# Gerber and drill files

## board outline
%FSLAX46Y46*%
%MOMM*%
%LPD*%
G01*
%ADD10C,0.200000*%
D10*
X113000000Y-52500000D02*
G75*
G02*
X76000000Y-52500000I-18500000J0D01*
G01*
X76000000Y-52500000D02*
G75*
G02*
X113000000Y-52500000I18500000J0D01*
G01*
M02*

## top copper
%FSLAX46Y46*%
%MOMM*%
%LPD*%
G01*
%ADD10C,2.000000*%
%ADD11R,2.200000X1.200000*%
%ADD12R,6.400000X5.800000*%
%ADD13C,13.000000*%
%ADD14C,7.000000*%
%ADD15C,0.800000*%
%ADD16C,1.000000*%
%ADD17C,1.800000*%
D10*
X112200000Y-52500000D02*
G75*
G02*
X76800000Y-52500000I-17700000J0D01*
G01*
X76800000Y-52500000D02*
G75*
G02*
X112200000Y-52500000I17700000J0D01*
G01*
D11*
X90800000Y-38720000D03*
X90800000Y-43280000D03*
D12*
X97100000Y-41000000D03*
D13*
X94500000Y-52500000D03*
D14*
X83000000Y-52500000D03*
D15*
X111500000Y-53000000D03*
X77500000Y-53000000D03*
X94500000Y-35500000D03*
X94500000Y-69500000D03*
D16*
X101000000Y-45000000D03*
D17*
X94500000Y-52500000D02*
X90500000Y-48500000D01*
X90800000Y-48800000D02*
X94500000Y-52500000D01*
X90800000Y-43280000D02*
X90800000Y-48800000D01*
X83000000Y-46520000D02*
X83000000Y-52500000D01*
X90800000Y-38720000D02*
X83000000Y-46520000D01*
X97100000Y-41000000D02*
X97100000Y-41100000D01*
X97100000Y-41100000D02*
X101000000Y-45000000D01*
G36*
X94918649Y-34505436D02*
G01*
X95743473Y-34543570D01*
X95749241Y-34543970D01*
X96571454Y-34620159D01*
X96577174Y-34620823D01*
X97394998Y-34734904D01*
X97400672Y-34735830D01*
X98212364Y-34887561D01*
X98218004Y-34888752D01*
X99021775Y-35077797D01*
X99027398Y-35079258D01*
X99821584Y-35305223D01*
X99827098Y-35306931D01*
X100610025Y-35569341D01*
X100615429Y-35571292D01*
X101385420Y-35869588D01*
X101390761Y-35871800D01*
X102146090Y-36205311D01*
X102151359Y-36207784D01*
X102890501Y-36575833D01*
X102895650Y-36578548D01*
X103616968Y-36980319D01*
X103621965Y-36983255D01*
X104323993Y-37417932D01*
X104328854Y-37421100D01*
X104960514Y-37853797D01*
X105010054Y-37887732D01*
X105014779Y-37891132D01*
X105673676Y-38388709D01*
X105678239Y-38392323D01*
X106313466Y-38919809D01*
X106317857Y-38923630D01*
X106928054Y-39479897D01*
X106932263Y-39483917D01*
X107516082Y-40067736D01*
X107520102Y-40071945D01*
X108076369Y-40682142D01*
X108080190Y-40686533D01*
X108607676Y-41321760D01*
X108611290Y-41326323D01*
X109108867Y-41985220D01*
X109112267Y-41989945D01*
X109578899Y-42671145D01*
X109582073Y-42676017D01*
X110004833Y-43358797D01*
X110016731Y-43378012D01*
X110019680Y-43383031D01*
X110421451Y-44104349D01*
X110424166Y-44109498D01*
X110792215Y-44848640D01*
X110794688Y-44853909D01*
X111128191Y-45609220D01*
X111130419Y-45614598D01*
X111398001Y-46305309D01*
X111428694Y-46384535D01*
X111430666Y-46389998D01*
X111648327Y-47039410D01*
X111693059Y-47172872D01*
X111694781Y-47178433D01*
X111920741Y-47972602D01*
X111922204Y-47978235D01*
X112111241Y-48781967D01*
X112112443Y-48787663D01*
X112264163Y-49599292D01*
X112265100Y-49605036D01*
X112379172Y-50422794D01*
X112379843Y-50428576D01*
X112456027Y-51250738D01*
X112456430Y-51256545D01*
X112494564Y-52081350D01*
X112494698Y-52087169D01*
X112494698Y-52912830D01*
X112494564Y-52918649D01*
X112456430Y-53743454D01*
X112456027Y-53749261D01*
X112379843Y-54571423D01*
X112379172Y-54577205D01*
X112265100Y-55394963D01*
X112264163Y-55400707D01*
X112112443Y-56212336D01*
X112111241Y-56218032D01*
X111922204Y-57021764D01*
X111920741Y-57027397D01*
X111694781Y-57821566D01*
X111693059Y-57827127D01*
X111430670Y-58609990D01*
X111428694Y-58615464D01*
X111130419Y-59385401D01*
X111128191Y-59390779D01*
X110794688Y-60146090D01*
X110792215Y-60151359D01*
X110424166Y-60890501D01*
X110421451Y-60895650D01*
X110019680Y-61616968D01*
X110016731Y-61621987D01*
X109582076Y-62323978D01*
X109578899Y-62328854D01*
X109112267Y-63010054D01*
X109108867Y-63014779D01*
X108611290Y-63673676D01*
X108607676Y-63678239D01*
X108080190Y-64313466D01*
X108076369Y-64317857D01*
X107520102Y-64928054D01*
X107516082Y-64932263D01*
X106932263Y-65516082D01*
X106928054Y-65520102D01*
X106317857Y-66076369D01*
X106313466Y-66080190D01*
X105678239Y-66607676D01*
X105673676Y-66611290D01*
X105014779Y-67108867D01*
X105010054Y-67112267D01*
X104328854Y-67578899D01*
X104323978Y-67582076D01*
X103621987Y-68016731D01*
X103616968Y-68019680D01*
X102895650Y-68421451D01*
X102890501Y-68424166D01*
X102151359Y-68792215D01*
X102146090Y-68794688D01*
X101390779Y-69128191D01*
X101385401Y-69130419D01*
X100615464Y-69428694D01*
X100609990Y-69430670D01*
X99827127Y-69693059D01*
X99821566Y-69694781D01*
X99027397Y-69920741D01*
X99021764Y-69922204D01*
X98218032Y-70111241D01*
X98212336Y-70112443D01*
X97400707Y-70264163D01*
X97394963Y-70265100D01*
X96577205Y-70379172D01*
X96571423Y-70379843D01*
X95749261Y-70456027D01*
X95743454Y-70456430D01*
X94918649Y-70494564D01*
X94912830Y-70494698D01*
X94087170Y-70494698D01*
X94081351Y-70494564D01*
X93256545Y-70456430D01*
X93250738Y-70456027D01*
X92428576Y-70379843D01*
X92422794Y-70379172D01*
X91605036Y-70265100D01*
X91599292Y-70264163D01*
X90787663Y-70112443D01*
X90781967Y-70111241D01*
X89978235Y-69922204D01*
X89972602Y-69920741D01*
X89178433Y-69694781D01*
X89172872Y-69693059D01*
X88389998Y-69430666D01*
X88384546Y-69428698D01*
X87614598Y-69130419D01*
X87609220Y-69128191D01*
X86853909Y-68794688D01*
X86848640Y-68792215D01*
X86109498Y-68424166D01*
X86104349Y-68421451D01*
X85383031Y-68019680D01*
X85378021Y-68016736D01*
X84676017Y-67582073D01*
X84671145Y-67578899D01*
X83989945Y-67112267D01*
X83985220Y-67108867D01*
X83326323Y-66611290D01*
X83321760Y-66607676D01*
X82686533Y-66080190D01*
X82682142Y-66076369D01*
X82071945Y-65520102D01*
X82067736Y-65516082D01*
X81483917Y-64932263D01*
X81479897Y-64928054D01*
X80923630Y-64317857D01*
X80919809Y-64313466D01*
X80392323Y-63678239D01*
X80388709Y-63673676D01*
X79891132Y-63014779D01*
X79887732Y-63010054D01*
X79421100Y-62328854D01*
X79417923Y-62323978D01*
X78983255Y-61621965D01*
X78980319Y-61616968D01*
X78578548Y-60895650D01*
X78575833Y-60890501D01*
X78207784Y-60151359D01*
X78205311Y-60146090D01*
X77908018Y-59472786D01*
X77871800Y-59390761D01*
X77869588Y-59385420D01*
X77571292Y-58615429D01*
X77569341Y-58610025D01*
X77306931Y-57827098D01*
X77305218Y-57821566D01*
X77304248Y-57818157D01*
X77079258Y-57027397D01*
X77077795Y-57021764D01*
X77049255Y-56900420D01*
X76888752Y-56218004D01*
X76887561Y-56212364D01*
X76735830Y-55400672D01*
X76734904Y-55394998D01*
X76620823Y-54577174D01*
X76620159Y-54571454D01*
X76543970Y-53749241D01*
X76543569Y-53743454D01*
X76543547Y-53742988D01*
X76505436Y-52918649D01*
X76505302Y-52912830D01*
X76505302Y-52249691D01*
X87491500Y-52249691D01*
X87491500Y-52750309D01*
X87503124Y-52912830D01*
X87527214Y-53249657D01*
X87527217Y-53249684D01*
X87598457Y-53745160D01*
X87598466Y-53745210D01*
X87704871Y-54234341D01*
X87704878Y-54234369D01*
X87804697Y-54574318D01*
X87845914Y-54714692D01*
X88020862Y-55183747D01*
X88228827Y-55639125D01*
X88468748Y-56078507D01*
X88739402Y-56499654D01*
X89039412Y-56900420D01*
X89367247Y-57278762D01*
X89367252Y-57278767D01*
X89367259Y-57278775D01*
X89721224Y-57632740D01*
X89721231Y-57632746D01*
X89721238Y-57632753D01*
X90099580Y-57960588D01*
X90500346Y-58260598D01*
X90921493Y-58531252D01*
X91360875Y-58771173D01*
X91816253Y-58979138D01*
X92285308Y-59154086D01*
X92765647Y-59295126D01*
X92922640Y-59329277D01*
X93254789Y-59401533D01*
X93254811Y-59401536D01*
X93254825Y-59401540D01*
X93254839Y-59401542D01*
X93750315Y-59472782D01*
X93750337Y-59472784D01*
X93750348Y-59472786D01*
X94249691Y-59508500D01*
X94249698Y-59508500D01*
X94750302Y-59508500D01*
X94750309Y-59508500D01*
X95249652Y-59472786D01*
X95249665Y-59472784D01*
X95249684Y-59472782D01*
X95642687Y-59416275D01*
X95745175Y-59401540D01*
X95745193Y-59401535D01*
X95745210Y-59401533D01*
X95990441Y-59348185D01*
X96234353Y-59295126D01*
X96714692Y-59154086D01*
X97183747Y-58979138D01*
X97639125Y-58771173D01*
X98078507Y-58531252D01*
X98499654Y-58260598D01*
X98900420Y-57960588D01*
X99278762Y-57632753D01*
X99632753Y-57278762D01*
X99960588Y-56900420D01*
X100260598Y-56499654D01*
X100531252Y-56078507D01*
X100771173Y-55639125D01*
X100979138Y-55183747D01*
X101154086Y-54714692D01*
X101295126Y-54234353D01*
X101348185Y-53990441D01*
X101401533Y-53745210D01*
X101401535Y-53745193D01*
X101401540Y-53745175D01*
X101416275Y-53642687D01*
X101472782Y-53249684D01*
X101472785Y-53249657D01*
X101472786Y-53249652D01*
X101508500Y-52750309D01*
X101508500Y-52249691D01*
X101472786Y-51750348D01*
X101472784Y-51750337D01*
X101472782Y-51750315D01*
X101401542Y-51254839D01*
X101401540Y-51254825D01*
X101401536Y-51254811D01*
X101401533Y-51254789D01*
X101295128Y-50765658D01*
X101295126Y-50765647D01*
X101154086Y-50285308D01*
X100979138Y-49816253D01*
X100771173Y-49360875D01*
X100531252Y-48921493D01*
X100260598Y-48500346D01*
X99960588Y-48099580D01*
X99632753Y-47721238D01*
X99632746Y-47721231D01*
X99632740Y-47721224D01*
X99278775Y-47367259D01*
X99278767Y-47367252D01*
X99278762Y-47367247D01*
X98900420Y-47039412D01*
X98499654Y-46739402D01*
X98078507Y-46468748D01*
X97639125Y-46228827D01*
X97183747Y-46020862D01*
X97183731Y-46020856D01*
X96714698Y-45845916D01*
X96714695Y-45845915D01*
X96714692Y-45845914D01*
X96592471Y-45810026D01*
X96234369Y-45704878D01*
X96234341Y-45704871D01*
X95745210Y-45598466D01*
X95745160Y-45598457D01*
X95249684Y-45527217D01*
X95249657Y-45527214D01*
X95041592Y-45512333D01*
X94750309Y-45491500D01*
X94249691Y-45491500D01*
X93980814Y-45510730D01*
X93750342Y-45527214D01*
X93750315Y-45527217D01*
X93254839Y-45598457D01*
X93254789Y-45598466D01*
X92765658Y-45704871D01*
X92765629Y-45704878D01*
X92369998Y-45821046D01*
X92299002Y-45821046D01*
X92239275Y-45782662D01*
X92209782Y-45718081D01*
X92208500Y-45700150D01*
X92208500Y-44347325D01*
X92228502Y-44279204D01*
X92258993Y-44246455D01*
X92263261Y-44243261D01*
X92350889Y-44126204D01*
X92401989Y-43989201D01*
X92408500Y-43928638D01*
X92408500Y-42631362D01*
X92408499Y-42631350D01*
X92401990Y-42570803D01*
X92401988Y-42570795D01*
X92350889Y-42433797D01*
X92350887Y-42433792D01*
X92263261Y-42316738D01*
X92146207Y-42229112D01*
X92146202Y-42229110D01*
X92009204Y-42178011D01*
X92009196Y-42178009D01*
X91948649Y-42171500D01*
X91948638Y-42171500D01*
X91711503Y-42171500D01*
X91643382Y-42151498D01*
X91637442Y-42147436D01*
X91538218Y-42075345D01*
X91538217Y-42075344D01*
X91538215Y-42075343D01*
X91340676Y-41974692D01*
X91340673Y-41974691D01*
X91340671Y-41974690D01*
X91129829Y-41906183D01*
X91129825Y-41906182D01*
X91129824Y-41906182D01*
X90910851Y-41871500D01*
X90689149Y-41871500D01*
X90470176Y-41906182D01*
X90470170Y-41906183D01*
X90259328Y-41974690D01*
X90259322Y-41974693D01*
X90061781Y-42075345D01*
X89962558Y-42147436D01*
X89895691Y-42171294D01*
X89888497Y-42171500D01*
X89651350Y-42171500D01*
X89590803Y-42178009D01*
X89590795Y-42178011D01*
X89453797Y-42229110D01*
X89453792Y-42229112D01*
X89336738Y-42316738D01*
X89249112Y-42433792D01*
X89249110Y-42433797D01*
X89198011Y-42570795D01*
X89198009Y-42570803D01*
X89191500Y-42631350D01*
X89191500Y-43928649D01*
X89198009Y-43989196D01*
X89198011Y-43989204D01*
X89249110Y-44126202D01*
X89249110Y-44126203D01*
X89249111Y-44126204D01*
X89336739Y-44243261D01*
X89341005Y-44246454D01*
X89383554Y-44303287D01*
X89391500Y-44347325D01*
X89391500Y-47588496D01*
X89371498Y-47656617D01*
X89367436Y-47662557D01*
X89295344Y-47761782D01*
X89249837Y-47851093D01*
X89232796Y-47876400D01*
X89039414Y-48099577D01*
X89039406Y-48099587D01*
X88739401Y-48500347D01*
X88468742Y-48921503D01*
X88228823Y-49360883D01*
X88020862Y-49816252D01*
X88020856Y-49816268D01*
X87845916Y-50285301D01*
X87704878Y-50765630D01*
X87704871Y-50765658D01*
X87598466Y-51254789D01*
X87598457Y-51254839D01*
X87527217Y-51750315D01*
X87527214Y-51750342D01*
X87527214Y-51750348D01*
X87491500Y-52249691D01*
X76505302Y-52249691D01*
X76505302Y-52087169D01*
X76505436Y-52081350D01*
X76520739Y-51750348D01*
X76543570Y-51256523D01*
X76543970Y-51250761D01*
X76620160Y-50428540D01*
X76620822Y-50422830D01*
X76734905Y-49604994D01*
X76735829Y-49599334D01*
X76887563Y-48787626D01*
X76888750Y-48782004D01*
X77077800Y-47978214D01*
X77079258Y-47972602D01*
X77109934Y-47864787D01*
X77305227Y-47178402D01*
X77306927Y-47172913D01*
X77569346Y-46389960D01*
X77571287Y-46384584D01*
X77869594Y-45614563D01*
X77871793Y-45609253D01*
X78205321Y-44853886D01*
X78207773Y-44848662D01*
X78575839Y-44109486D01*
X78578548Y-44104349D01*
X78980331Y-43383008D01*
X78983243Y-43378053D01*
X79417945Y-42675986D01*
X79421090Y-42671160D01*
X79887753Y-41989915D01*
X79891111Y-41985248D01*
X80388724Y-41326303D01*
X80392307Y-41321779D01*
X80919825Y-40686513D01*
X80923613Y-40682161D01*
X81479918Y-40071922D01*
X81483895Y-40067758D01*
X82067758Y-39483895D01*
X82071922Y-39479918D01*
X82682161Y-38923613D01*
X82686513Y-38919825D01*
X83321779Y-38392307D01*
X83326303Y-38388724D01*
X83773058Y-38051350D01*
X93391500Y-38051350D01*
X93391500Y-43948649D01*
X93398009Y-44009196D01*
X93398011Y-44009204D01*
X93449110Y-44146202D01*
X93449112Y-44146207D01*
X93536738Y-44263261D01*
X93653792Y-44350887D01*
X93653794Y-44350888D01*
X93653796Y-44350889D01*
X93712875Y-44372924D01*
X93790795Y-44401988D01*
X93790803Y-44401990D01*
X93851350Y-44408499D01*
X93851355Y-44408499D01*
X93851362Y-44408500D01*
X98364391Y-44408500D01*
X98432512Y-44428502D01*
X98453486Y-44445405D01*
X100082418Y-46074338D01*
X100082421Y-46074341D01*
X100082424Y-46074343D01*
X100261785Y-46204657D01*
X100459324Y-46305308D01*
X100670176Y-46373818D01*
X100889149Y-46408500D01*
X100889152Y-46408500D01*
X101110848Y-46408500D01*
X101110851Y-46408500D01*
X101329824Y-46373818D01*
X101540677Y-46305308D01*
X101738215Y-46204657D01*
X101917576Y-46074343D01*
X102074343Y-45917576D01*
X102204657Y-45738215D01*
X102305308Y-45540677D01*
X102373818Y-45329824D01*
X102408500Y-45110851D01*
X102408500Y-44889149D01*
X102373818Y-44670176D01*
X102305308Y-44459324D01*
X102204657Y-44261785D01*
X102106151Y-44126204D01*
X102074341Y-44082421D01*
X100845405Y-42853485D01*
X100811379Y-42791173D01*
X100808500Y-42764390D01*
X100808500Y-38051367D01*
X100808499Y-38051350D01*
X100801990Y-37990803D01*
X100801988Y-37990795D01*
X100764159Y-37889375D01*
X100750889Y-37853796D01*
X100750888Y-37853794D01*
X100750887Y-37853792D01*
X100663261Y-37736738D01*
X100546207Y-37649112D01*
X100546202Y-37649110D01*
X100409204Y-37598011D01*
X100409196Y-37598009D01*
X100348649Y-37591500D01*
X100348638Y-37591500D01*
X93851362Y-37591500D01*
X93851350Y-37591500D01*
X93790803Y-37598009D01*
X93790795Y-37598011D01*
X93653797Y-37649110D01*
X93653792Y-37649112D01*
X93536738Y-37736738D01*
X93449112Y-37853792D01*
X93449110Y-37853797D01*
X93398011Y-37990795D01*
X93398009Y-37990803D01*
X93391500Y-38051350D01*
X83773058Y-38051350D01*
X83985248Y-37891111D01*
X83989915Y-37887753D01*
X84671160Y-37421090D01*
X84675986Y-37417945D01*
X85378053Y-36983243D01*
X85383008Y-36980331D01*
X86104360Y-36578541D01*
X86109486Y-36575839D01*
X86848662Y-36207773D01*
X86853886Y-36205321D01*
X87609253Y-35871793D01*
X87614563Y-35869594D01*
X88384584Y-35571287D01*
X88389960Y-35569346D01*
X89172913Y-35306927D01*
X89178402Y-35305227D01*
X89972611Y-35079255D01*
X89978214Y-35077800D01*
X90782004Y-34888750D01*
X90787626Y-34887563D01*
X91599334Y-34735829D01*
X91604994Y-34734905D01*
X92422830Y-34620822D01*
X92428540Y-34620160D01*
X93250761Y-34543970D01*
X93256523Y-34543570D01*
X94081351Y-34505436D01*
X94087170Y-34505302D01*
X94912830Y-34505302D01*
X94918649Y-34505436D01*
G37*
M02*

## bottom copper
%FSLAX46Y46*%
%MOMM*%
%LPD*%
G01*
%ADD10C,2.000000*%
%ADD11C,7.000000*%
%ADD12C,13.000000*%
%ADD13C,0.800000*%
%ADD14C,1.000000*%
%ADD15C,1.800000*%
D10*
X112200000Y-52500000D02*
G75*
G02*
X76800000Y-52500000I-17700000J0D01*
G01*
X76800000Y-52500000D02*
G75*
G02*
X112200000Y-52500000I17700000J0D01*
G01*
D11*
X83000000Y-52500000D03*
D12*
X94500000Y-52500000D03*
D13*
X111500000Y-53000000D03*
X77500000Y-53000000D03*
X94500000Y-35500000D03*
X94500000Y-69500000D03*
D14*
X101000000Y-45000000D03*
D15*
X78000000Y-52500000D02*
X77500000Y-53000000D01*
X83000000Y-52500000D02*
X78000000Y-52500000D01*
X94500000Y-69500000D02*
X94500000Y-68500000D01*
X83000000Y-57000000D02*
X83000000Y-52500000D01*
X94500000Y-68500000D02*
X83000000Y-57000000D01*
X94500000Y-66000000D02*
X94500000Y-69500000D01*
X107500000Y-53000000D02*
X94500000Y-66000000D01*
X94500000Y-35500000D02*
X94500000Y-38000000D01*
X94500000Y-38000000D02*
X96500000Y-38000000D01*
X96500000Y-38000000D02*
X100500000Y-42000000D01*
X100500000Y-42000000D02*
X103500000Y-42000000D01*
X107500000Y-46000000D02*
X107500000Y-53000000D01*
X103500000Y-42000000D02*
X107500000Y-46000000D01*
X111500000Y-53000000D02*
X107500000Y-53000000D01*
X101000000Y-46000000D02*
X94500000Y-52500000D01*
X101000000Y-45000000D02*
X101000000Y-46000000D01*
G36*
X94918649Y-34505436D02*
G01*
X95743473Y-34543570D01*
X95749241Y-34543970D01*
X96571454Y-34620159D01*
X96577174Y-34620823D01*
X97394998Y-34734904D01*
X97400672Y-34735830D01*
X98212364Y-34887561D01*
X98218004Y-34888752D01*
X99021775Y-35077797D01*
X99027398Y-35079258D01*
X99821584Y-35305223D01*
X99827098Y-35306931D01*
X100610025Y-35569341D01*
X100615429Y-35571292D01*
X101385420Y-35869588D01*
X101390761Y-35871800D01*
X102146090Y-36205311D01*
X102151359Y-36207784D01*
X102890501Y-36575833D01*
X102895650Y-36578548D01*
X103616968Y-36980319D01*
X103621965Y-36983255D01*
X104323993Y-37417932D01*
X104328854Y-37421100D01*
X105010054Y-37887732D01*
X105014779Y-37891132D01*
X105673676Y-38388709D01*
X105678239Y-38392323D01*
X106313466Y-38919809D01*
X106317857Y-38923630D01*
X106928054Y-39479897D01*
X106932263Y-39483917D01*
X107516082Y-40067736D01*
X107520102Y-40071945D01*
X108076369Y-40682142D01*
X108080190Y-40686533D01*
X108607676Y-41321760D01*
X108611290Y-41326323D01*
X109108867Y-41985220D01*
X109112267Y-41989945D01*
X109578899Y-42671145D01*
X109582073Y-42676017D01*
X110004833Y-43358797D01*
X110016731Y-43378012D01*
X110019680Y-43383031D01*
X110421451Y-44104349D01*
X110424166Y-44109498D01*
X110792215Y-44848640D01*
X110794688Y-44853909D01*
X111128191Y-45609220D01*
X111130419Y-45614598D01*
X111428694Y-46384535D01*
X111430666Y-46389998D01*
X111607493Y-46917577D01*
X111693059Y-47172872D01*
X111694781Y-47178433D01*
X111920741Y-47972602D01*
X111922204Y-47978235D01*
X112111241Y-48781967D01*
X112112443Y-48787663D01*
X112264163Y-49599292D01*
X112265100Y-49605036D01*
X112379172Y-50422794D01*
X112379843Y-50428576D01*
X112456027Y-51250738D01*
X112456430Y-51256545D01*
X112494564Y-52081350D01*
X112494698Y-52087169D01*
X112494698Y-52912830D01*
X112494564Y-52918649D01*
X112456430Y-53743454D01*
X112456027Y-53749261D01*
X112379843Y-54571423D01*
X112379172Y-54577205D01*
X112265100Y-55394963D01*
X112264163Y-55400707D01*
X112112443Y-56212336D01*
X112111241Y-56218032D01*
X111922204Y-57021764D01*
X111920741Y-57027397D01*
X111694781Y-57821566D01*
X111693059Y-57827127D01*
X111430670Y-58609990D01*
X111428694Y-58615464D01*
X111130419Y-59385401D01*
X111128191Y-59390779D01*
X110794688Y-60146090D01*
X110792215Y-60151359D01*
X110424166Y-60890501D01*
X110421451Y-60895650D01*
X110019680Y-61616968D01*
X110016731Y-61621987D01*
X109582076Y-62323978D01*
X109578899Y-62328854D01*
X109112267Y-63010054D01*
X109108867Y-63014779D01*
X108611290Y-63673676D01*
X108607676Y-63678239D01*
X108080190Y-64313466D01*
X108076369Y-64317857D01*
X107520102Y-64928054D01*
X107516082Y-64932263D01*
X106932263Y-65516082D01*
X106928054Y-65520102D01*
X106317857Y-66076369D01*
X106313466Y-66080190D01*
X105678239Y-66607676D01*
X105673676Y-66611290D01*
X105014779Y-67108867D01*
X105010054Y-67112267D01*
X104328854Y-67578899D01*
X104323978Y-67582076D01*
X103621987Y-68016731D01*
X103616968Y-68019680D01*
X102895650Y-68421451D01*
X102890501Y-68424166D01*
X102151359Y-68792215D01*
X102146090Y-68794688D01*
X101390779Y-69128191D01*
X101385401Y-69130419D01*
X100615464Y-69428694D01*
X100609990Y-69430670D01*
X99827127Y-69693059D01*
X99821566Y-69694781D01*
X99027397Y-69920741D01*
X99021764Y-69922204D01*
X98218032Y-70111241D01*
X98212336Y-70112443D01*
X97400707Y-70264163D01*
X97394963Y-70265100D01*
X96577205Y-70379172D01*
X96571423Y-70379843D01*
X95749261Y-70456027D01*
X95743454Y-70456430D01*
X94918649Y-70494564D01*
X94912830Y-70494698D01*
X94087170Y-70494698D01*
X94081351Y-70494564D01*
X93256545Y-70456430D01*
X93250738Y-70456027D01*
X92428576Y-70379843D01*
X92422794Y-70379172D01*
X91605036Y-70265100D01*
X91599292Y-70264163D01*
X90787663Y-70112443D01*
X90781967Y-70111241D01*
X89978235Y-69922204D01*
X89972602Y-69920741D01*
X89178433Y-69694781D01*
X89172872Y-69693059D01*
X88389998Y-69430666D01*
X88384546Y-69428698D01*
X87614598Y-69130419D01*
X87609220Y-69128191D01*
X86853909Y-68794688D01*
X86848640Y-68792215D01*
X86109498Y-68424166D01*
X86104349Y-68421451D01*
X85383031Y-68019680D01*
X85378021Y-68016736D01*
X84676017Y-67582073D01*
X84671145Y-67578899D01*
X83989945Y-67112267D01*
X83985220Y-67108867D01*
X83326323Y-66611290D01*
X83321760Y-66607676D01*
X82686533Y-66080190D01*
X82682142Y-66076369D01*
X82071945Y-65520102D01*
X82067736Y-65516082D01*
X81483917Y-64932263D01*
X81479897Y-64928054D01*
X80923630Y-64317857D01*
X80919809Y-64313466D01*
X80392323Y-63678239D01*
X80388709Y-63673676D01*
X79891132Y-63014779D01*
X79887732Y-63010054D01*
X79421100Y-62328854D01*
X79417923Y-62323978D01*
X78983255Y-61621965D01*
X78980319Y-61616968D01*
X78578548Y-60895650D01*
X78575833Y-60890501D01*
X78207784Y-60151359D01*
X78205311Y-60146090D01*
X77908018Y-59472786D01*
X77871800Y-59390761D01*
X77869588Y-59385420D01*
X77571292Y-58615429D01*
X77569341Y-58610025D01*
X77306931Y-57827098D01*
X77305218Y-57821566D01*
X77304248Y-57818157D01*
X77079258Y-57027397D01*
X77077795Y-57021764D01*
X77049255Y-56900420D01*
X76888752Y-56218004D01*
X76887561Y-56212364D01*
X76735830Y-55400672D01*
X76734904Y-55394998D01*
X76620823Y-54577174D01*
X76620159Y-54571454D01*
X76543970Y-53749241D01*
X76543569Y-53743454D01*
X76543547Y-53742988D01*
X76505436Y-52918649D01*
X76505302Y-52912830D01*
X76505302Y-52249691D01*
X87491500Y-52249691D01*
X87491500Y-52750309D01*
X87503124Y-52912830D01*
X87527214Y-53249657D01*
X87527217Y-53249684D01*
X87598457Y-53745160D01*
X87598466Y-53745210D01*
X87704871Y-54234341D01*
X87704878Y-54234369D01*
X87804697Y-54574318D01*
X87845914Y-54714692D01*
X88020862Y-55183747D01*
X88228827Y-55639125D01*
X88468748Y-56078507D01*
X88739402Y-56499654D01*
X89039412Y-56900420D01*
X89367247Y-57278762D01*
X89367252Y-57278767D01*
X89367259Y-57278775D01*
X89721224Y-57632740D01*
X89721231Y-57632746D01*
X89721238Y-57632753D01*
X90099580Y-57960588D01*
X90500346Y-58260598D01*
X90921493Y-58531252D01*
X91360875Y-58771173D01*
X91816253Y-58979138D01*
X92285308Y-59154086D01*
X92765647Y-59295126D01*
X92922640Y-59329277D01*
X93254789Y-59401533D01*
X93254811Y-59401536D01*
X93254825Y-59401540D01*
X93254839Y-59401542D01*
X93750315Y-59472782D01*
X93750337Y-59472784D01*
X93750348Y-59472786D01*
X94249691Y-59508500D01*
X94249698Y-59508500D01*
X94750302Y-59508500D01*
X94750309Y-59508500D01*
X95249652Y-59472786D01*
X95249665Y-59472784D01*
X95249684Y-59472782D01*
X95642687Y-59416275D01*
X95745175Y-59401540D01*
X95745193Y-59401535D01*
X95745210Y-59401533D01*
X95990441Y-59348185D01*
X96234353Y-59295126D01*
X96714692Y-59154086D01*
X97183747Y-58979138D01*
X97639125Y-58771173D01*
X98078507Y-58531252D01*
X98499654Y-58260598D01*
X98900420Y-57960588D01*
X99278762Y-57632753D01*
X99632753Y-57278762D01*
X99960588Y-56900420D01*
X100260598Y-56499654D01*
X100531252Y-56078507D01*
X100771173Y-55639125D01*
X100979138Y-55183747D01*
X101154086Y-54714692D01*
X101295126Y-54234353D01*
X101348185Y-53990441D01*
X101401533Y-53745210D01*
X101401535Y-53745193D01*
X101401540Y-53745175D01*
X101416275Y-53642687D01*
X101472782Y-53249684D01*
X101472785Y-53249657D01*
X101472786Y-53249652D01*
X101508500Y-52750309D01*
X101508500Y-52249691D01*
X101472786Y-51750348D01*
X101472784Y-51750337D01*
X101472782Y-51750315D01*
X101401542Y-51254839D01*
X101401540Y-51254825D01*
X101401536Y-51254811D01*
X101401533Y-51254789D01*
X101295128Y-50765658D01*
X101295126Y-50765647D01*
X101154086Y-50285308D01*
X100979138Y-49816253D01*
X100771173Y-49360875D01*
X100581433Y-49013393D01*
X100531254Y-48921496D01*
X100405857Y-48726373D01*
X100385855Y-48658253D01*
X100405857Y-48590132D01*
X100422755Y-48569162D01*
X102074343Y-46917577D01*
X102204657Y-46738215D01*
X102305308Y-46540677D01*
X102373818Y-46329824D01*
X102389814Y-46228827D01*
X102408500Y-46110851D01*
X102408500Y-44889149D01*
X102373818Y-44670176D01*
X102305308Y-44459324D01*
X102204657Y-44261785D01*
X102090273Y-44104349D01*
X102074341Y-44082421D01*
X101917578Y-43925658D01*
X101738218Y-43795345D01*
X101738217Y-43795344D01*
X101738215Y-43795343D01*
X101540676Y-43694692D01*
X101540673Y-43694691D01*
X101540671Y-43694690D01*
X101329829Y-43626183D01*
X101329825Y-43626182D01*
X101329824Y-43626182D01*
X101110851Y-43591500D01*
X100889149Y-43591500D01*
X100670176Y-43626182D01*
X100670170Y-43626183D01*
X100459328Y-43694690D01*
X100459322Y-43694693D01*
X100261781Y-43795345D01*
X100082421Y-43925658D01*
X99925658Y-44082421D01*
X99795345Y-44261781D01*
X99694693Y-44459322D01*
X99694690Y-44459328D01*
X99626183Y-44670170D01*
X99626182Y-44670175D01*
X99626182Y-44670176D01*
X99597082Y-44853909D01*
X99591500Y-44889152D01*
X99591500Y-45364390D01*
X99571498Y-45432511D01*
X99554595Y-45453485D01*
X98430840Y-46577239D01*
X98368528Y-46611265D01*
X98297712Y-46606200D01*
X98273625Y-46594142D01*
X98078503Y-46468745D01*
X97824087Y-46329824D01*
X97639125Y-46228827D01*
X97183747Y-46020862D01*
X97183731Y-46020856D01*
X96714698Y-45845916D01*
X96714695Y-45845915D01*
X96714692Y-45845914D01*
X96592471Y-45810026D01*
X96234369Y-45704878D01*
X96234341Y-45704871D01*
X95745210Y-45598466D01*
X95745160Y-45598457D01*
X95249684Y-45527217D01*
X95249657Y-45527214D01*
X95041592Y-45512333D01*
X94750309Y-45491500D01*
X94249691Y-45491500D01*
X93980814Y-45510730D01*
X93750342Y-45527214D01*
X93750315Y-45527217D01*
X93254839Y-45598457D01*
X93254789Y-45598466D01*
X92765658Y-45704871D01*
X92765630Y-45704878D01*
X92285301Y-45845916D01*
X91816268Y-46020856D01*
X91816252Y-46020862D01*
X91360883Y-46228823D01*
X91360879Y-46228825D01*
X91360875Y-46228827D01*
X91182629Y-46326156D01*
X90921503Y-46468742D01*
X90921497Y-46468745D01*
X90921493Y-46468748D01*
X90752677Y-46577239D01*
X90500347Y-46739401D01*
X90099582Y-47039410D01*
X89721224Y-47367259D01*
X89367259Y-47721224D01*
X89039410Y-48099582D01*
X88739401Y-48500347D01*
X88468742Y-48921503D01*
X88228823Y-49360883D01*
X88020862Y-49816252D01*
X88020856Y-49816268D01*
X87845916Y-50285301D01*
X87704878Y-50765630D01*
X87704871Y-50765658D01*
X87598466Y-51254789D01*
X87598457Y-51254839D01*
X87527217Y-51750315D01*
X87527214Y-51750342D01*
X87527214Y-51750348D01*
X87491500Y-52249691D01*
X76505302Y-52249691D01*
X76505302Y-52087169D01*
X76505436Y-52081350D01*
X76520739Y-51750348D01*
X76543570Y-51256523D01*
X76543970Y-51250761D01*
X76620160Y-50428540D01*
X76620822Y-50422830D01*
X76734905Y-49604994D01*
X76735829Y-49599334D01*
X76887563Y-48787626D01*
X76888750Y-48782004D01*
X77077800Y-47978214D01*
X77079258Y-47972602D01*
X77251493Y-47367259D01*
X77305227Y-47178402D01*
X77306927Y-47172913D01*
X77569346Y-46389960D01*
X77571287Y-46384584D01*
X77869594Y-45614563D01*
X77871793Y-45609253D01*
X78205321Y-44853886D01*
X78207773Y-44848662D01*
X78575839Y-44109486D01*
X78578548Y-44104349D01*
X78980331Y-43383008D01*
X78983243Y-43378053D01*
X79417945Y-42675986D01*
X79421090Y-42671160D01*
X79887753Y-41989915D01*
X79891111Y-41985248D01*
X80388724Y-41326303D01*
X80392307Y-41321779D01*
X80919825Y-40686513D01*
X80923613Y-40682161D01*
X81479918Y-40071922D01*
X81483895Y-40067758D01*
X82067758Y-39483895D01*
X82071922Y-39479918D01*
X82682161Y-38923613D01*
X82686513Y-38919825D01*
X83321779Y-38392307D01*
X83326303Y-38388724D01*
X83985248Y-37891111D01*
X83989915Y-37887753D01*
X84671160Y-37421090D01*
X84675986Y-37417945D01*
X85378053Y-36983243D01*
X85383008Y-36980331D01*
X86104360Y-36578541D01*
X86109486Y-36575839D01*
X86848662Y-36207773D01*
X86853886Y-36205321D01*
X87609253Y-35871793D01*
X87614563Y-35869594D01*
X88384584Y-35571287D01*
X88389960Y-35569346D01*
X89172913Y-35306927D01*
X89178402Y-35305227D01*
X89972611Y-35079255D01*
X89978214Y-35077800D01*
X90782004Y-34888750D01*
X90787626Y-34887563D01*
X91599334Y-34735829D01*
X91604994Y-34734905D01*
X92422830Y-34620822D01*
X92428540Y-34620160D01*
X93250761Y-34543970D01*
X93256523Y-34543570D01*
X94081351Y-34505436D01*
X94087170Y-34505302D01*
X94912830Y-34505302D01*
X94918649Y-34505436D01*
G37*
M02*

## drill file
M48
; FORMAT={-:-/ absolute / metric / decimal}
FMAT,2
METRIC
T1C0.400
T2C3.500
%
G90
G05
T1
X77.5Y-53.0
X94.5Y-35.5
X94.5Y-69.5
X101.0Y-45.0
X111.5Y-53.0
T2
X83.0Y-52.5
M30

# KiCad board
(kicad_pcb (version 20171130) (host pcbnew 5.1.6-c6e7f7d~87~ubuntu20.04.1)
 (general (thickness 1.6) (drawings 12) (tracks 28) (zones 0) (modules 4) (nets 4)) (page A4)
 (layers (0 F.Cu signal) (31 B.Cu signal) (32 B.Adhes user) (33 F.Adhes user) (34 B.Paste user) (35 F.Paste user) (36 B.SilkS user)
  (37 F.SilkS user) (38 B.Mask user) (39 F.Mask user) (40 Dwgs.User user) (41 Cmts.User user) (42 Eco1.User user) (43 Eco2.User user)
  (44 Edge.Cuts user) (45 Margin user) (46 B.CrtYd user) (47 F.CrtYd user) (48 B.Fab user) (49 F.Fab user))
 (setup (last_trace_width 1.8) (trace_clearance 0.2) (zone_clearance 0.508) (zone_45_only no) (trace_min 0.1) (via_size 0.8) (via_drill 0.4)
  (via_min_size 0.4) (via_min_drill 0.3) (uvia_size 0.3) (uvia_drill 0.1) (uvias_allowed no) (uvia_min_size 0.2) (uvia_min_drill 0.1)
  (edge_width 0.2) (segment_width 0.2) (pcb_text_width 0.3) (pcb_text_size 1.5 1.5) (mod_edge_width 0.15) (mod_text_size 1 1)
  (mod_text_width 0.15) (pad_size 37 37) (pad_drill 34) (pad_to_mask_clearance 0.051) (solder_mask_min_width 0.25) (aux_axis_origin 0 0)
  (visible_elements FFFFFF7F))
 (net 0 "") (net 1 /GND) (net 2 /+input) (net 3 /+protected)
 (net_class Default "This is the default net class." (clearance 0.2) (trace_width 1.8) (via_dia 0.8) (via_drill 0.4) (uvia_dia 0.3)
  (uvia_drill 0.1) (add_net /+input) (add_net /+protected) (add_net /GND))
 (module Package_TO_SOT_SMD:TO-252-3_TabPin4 (layer F.Cu) (at 95 41)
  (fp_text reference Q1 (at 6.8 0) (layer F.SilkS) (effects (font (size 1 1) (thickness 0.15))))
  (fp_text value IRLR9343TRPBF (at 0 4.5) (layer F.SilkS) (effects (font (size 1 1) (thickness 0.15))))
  (pad 1 smd rect (at -4.2 -2.28) (size 2.2 1.2) (layers F.Cu F.Paste F.Mask) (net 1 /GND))
  (pad 3 smd rect (at -4.2 2.28) (size 2.2 1.2) (layers F.Cu F.Paste F.Mask) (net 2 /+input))
  (pad 4 smd rect (at 2.1 0) (size 6.4 5.8) (layers F.Cu F.Mask) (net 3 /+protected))
  (pad "" smd rect (at 3.775 1.525) (size 3.05 2.75) (layers F.Paste))
  (pad "" smd rect (at 0.425 -1.525) (size 3.05 2.75) (layers F.Paste))
  (pad "" smd rect (at 3.775 -1.525) (size 3.05 2.75) (layers F.Paste))
  (pad "" smd rect (at 0.425 1.525) (size 3.05 2.75) (layers F.Paste)))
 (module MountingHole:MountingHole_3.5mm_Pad (layer F.Cu) (at 94.5 52.5)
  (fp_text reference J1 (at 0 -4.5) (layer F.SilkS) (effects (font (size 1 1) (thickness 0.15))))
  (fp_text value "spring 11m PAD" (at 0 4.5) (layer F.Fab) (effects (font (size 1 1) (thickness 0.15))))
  (pad 1 smd circle (at 0 0) (size 13 13) (layers F.Cu F.Paste F.Mask) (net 2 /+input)))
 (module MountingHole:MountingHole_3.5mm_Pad (layer F.Cu) (at 83 52.5)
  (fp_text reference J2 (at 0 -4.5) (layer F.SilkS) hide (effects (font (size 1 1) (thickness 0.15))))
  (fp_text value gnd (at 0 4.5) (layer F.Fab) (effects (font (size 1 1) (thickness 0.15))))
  (pad 1 thru_hole circle (at 0 0) (size 7 7) (drill 3.5) (layers *.Cu *.Mask) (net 1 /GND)))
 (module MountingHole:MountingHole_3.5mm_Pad (layer F.Cu) (at 94.5 52.5)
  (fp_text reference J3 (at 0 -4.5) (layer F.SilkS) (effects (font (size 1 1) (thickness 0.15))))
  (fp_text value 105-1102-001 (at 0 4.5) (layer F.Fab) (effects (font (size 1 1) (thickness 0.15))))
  (pad 1 smd circle (at 0 0) (size 13 13) (layers B.Cu B.Paste B.Mask) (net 3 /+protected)))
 (gr_circle (center 94.5 52.5) (end 112.2 52.5) (layer F.Cu) (width 2))
 (gr_circle (center 94.5 52.5) (end 112.2 52.5) (layer B.Cu) (width 2))
 (gr_circle (center 94.5 52.5) (end 113 52.5) (layer Edge.Cuts) (width 0.2))
 (via (at 111.5 53) (size 0.8) (drill 0.4) (layers F.Cu B.Cu) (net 1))
 (via (at 77.5 53) (size 0.8) (drill 0.4) (layers F.Cu B.Cu) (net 1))
 (via (at 94.5 35.5) (size 0.8) (drill 0.4) (layers F.Cu B.Cu) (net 1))
 (via (at 94.5 69.5) (size 0.8) (drill 0.4) (layers F.Cu B.Cu) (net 1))
 (segment (start 94.5 52.5) (end 90.5 48.5) (width 1.8) (layer F.Cu) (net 2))
 (segment (start 90.8 48.8) (end 94.5 52.5) (width 1.8) (layer F.Cu) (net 2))
 (segment (start 90.8 43.28) (end 90.8 48.8) (width 1.8) (layer F.Cu) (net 2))
 (segment (start 83 46.52) (end 83 52.5) (width 1.8) (layer F.Cu) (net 1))
 (segment (start 90.8 38.72) (end 83 46.52) (width 1.8) (layer F.Cu) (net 1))
 (segment (start 78 52.5) (end 77.5 53) (width 1.8) (layer B.Cu) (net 1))
 (segment (start 83 52.5) (end 78 52.5) (width 1.8) (layer B.Cu) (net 1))
 (segment (start 94.5 69.5) (end 94.5 68.5) (width 1.8) (layer B.Cu) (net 1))
 (segment (start 83 57) (end 83 52.5) (width 1.8) (layer B.Cu) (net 1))
 (segment (start 94.5 68.5) (end 83 57) (width 1.8) (layer B.Cu) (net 1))
 (segment (start 94.5 66) (end 94.5 69.5) (width 1.8) (layer B.Cu) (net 1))
 (segment (start 107.5 53) (end 94.5 66) (width 1.8) (layer B.Cu) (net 1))
 (segment (start 94.5 35.5) (end 94.5 38) (width 1.8) (layer B.Cu) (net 1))
 (segment (start 94.5 38) (end 96.5 38) (width 1.8) (layer B.Cu) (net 1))
 (segment (start 96.5 38) (end 100.5 42) (width 1.8) (layer B.Cu) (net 1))
 (segment (start 100.5 42) (end 103.5 42) (width 1.8) (layer B.Cu) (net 1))
 (segment (start 107.5 46) (end 107.5 53) (width 1.8) (layer B.Cu) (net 1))
 (segment (start 103.5 42) (end 107.5 46) (width 1.8) (layer B.Cu) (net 1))
 (segment (start 111.5 53) (end 107.5 53) (width 1.8) (layer B.Cu) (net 1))
 (segment (start 97.1 41) (end 97.1 41.1) (width 1.8) (layer F.Cu) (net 3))
 (via (at 101 45) (size 1) (drill 0.4) (layers F.Cu B.Cu) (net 3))
 (segment (start 97.1 41.1) (end 101 45) (width 1.8) (layer F.Cu) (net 3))
 (segment (start 101 46) (end 94.5 52.5) (width 1.8) (layer B.Cu) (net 3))
 (segment (start 101 45) (end 101 46) (width 1.8) (layer B.Cu) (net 3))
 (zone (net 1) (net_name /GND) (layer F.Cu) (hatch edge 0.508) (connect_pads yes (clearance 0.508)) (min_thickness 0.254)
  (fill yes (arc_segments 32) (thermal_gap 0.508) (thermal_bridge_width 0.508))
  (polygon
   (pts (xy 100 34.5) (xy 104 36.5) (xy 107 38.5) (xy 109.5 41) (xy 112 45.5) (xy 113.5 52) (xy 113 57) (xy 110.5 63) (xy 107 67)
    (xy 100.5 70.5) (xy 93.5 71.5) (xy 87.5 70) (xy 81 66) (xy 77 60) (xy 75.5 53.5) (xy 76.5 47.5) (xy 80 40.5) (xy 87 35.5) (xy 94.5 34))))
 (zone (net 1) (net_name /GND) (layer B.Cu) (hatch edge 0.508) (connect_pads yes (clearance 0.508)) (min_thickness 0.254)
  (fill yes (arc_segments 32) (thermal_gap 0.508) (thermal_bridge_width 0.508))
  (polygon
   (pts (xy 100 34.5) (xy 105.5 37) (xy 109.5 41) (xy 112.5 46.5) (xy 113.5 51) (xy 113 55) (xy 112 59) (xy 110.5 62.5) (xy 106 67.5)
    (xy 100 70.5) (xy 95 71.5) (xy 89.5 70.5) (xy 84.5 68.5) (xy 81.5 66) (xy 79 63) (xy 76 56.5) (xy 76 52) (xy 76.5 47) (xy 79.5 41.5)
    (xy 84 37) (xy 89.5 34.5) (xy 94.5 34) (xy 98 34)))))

